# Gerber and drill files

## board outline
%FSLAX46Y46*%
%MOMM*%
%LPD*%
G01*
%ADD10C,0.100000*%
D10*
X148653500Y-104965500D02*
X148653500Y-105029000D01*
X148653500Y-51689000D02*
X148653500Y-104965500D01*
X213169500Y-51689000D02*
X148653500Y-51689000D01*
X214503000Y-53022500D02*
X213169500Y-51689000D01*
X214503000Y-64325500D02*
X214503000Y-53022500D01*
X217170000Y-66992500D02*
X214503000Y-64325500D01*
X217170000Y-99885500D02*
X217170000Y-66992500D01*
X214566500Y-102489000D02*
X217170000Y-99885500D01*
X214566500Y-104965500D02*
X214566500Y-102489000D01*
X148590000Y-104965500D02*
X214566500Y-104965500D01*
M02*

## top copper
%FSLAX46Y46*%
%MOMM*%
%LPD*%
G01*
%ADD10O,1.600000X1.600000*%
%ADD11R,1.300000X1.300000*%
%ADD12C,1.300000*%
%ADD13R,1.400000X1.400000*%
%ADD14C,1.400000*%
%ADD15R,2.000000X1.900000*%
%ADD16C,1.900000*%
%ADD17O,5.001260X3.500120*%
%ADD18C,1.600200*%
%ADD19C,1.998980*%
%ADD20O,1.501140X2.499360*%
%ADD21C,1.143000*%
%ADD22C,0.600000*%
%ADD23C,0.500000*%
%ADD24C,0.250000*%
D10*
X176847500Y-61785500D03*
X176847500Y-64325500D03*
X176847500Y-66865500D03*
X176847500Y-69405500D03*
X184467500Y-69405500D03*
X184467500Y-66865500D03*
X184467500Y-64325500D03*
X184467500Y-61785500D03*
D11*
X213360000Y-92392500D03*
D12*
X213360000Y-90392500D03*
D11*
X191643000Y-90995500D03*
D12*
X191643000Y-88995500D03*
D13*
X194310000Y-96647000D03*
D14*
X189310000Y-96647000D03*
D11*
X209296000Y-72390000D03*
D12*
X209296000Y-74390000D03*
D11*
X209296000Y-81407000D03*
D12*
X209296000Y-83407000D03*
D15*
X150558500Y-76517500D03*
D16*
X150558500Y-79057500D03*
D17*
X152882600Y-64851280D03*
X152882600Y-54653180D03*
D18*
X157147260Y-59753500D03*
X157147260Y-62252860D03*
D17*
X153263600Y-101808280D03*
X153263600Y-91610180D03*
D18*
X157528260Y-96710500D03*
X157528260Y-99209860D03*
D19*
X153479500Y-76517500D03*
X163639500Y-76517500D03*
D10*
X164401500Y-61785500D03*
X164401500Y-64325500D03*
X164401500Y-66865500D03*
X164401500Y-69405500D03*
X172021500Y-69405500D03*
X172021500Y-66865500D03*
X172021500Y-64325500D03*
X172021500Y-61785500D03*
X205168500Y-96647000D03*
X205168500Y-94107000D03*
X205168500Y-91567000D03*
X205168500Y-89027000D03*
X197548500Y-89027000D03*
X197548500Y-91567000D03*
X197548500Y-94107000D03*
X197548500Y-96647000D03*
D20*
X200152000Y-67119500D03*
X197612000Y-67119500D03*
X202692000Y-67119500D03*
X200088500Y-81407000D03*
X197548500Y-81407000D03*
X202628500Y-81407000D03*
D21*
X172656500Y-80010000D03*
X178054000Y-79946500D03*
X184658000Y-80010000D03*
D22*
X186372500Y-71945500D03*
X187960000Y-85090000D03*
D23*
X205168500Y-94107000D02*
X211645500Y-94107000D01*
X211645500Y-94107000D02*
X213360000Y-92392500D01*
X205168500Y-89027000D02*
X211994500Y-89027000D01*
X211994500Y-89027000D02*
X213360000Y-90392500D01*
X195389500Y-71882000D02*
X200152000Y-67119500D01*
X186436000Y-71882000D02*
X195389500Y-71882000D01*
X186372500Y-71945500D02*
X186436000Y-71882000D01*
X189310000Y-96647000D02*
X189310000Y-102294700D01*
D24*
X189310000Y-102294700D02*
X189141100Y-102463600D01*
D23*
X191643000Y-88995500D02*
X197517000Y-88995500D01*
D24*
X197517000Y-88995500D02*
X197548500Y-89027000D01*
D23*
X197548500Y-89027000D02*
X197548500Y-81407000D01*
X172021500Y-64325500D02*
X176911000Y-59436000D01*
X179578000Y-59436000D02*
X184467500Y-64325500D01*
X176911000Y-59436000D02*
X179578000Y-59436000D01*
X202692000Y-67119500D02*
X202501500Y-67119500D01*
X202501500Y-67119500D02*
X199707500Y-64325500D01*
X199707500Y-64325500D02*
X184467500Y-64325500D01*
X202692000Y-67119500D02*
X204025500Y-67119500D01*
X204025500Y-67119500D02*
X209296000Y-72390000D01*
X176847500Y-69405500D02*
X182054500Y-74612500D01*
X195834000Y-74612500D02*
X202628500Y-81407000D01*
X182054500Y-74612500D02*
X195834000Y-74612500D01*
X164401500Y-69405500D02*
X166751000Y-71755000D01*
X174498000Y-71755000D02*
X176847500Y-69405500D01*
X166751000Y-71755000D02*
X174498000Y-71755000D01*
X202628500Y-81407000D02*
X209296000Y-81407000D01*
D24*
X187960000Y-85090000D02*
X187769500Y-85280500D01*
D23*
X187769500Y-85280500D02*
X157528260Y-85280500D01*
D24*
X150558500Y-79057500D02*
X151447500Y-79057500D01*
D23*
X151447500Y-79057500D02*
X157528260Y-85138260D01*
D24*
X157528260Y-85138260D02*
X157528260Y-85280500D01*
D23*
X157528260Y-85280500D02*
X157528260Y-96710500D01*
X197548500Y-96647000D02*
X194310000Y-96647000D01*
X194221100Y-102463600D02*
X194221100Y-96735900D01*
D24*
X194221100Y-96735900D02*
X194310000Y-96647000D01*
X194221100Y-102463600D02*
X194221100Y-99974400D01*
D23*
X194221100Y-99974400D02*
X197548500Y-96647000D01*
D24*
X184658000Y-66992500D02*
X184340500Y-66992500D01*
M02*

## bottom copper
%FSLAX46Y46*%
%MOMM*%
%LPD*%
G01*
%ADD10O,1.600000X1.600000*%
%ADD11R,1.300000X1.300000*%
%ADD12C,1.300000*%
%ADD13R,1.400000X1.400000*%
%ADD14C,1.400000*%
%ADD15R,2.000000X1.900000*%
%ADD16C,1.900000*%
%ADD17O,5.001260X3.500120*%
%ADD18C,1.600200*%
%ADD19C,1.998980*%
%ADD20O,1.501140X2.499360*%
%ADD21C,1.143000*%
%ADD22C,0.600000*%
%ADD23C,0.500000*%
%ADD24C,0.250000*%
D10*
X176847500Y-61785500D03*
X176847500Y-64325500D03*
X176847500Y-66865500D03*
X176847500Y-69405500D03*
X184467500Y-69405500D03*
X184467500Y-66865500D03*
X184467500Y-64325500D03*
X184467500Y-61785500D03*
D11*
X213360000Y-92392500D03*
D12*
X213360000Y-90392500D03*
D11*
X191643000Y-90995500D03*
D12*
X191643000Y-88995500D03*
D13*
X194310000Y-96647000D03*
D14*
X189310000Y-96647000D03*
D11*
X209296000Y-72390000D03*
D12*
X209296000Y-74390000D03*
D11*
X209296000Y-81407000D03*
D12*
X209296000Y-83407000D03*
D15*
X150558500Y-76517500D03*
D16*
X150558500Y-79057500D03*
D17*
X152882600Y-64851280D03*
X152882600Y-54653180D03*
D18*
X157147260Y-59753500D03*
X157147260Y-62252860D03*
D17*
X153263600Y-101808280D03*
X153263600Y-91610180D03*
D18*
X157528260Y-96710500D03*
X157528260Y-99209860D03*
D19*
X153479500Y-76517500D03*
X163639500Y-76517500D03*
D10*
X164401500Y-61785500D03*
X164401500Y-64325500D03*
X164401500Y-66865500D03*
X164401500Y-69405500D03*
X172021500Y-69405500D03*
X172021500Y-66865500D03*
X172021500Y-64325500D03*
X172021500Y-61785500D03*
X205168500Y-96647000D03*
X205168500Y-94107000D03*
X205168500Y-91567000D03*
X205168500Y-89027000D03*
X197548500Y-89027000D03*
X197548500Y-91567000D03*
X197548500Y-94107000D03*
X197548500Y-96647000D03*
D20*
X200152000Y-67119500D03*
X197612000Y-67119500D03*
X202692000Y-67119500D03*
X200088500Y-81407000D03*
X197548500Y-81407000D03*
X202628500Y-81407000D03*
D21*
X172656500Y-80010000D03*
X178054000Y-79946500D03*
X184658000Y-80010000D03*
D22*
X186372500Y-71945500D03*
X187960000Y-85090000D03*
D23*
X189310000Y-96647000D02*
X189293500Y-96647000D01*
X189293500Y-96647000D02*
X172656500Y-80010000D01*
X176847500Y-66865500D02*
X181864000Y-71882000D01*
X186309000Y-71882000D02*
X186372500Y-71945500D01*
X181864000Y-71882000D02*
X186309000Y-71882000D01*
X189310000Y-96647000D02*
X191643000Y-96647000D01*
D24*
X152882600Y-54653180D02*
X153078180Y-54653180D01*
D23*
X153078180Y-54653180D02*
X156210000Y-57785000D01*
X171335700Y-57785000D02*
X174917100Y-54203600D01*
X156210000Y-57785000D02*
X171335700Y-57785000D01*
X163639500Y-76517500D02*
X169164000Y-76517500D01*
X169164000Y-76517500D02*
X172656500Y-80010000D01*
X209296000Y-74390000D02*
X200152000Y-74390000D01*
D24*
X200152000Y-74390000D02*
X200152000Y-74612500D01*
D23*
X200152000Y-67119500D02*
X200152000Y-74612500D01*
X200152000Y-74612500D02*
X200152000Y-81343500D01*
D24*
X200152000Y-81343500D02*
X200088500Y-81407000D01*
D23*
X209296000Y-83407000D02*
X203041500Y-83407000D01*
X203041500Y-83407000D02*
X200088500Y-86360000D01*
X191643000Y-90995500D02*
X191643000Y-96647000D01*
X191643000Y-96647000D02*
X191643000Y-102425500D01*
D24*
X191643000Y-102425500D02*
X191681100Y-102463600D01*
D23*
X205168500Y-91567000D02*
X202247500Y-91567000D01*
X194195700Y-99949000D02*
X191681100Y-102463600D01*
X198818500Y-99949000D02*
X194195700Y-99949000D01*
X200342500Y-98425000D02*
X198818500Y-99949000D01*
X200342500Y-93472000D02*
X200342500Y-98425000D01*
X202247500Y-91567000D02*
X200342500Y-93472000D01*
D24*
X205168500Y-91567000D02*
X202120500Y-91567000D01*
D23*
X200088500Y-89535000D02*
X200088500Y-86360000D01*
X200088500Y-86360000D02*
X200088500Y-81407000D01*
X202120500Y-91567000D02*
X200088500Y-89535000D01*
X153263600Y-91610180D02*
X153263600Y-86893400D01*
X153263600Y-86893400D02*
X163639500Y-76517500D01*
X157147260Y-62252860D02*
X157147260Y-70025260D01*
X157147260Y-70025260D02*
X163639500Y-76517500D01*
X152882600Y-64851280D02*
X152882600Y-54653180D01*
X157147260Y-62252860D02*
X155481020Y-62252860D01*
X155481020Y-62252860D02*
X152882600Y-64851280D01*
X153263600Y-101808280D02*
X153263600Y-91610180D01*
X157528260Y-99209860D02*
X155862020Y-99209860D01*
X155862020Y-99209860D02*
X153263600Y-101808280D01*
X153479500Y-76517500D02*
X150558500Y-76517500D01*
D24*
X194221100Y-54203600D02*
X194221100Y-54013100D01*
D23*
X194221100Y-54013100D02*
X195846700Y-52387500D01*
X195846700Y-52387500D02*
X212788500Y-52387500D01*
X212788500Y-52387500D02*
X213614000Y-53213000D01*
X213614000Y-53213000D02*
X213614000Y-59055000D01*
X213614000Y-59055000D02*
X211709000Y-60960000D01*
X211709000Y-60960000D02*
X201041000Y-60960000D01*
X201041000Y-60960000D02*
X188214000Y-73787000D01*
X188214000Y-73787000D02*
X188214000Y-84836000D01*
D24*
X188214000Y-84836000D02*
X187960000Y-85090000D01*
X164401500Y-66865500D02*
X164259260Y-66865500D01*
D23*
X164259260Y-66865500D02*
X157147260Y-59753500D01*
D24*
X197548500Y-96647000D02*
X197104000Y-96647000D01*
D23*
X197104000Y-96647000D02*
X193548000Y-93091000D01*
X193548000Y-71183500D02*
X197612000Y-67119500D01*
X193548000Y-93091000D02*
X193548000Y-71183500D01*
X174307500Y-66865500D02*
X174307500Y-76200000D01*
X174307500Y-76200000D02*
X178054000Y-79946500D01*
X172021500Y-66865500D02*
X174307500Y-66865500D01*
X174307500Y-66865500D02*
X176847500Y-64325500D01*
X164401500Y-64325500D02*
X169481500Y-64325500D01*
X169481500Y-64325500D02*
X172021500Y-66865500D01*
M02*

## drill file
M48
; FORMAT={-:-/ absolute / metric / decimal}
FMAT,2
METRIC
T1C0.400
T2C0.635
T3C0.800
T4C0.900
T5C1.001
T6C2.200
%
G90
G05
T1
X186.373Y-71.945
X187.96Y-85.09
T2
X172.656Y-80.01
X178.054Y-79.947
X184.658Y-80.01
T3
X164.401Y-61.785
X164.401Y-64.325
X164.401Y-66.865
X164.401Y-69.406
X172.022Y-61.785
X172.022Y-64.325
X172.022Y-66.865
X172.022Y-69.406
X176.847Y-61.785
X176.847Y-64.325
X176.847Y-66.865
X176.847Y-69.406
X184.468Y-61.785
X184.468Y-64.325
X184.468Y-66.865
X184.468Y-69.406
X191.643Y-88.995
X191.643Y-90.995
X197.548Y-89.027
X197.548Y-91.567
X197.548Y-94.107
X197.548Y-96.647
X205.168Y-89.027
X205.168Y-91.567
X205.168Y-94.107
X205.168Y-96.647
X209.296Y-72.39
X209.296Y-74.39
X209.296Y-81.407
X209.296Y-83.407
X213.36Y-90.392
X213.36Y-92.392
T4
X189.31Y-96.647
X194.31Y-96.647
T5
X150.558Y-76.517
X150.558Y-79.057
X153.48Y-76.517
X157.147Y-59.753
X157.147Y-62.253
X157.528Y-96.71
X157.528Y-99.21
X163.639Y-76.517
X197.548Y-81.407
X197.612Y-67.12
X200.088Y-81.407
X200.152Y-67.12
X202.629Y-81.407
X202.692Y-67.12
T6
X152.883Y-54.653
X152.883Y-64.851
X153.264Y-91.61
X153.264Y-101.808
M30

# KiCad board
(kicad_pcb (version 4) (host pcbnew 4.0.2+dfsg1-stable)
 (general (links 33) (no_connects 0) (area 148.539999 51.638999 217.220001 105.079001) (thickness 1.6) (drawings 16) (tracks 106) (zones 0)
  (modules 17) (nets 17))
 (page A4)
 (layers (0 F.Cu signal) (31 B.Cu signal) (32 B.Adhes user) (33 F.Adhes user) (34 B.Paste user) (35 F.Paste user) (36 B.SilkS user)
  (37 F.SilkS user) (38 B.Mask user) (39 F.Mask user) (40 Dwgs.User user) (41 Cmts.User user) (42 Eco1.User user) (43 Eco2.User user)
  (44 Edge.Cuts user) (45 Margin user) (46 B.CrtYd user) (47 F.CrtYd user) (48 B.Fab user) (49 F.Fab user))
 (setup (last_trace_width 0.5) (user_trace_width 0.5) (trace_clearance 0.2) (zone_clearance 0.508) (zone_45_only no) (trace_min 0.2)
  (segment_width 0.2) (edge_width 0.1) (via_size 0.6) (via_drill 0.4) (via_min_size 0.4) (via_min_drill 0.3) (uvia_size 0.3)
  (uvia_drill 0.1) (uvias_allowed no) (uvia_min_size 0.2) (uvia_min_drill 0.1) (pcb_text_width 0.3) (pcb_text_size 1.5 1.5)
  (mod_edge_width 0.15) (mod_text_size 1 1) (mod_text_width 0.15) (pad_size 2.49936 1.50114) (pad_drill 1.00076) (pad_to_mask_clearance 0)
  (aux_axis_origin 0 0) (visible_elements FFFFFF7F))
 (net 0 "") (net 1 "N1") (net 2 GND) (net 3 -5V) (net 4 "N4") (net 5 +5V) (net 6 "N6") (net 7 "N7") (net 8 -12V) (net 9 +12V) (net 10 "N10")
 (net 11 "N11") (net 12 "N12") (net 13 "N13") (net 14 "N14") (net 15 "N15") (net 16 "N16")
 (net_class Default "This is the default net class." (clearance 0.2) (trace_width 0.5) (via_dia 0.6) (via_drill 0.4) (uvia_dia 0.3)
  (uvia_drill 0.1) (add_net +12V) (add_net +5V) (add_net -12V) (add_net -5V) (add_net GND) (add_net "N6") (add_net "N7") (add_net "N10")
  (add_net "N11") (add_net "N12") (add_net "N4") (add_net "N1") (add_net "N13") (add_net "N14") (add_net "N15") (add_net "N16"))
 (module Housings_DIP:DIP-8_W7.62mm (layer F.Cu) (at 176.8475 61.7855)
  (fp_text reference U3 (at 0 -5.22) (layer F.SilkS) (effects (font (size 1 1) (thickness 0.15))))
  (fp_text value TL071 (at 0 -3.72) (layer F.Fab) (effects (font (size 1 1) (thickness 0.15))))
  (pad 1 thru_hole oval (at 0 0) (size 1.6 1.6) (drill 0.8) (layers *.Cu *.Mask F.SilkS))
  (pad 2 thru_hole oval (at 0 2.54) (size 1.6 1.6) (drill 0.8) (layers *.Cu *.Mask F.SilkS) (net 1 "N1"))
  (pad 3 thru_hole oval (at 0 5.08) (size 1.6 1.6) (drill 0.8) (layers *.Cu *.Mask F.SilkS) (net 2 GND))
  (pad 4 thru_hole oval (at 0 7.62) (size 1.6 1.6) (drill 0.8) (layers *.Cu *.Mask F.SilkS) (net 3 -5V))
  (pad 5 thru_hole oval (at 7.62 7.62) (size 1.6 1.6) (drill 0.8) (layers *.Cu *.Mask F.SilkS))
  (pad 6 thru_hole oval (at 7.62 5.08) (size 1.6 1.6) (drill 0.8) (layers *.Cu *.Mask F.SilkS) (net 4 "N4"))
  (pad 7 thru_hole oval (at 7.62 2.54) (size 1.6 1.6) (drill 0.8) (layers *.Cu *.Mask F.SilkS) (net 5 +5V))
  (pad 8 thru_hole oval (at 7.62 0) (size 1.6 1.6) (drill 0.8) (layers *.Cu *.Mask F.SilkS)))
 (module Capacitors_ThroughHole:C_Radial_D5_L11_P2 (layer F.Cu) (at 213.36 92.3925 90)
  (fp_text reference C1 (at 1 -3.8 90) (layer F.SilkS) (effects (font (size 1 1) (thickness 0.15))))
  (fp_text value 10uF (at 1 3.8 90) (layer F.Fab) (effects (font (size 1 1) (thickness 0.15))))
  (pad 1 thru_hole rect (at 0 0 90) (size 1.3 1.3) (drill 0.8) (layers *.Cu *.Mask F.SilkS) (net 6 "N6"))
  (pad 2 thru_hole circle (at 2 0 90) (size 1.3 1.3) (drill 0.8) (layers *.Cu *.Mask F.SilkS) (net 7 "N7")))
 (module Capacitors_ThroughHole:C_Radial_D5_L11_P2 (layer F.Cu) (at 191.643 90.9955 90)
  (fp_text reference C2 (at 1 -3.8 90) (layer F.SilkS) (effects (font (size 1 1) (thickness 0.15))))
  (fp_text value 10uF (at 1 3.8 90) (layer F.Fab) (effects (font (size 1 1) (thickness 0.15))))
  (pad 1 thru_hole rect (at 0 0 90) (size 1.3 1.3) (drill 0.8) (layers *.Cu *.Mask F.SilkS) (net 2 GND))
  (pad 2 thru_hole circle (at 2 0 90) (size 1.3 1.3) (drill 0.8) (layers *.Cu *.Mask F.SilkS) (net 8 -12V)))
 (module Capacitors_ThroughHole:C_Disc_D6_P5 (layer F.Cu) (at 194.31 96.647 180)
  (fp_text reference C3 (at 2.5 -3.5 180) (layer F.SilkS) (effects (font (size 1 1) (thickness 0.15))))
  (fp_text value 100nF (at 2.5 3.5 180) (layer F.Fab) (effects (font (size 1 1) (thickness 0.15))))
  (pad 1 thru_hole rect (at 0 0 180) (size 1.4 1.4) (drill 0.9) (layers *.Cu *.Mask F.SilkS) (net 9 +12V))
  (pad 2 thru_hole circle (at 5 0 180) (size 1.4 1.4) (drill 0.9) (layers *.Cu *.Mask F.SilkS) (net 2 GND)))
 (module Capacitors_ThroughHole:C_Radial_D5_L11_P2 (layer F.Cu) (at 209.296 72.39 270)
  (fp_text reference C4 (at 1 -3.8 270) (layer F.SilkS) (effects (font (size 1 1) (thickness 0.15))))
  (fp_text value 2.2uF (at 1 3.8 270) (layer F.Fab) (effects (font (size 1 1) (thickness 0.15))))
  (pad 1 thru_hole rect (at 0 0 270) (size 1.3 1.3) (drill 0.8) (layers *.Cu *.Mask F.SilkS) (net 5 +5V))
  (pad 2 thru_hole circle (at 2 0 270) (size 1.3 1.3) (drill 0.8) (layers *.Cu *.Mask F.SilkS) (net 2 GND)))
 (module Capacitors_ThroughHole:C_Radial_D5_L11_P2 (layer F.Cu) (at 209.296 81.407 270)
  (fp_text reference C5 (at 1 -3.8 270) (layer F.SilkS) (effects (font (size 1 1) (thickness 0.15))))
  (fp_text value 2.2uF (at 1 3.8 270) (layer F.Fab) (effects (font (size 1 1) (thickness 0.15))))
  (pad 1 thru_hole rect (at 0 0 270) (size 1.3 1.3) (drill 0.8) (layers *.Cu *.Mask F.SilkS) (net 3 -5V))
  (pad 2 thru_hole circle (at 2 0 270) (size 1.3 1.3) (drill 0.8) (layers *.Cu *.Mask F.SilkS) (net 2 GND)))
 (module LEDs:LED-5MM (layer F.Cu) (at 150.5585 76.5175 270)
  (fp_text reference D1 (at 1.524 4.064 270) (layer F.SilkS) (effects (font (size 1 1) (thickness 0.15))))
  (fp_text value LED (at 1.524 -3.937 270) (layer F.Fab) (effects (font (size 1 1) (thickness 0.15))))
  (pad 1 thru_hole rect (at 0 0) (size 2 1.9) (drill 1.00076) (layers *.Cu *.Mask F.SilkS) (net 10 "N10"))
  (pad 2 thru_hole circle (at 2.54 0 270) (size 1.9 1.9) (drill 1.00076) (layers *.Cu *.Mask F.SilkS) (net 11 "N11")))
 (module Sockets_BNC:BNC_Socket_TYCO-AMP (layer F.Cu) (at 152.146 59.7535 90)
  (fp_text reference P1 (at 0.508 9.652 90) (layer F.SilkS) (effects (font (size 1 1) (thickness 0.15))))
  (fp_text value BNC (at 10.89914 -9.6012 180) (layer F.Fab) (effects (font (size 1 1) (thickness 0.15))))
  (pad 2 thru_hole oval (at -5.09778 0.7366 90) (size 3.50012 5.00126) (drill 2.19964) (layers *.Cu *.Mask F.SilkS) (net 2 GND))
  (pad 2 thru_hole oval (at 5.10032 0.7366 90) (size 3.50012 5.00126) (drill 2.19964) (layers *.Cu *.Mask F.SilkS) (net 2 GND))
  (pad 1 thru_hole circle (at 0 5.00126 90) (size 1.6002 1.6002) (drill 1.00076) (layers *.Cu *.Mask F.SilkS) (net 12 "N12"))
  (pad 2 thru_hole circle (at -2.49936 5.00126 90) (size 1.6002 1.6002) (drill 1.00076) (layers *.Cu *.Mask F.SilkS) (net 2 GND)))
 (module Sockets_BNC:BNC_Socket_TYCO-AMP (layer F.Cu) (at 152.527 96.7105 90)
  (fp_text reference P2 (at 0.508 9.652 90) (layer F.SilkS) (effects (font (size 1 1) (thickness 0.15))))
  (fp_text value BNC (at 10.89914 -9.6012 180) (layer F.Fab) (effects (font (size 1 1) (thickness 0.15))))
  (pad 2 thru_hole oval (at -5.09778 0.7366 90) (size 3.50012 5.00126) (drill 2.19964) (layers *.Cu *.Mask F.SilkS) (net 2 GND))
  (pad 2 thru_hole oval (at 5.10032 0.7366 90) (size 3.50012 5.00126) (drill 2.19964) (layers *.Cu *.Mask F.SilkS) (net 2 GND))
  (pad 1 thru_hole circle (at 0 5.00126 90) (size 1.6002 1.6002) (drill 1.00076) (layers *.Cu *.Mask F.SilkS) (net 11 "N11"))
  (pad 2 thru_hole circle (at -2.49936 5.00126 90) (size 1.6002 1.6002) (drill 1.00076) (layers *.Cu *.Mask F.SilkS) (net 2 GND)))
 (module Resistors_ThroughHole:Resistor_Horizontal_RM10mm (layer F.Cu) (at 153.4795 76.5175)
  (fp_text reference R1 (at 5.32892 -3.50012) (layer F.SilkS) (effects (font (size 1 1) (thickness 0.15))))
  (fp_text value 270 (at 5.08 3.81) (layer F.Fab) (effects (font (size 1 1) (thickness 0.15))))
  (pad 1 thru_hole circle (at 0 0) (size 1.99898 1.99898) (drill 1.00076) (layers *.Cu *.SilkS *.Mask) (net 10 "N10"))
  (pad 2 thru_hole circle (at 10.16 0) (size 1.99898 1.99898) (drill 1.00076) (layers *.Cu *.SilkS *.Mask) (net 2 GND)))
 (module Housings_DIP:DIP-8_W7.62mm (layer F.Cu) (at 164.4015 61.7855)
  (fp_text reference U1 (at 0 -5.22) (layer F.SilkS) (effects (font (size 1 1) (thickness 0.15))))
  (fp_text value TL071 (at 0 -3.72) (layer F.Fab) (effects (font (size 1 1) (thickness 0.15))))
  (pad 1 thru_hole oval (at 0 0) (size 1.6 1.6) (drill 0.8) (layers *.Cu *.Mask F.SilkS))
  (pad 2 thru_hole oval (at 0 2.54) (size 1.6 1.6) (drill 0.8) (layers *.Cu *.Mask F.SilkS) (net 1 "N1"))
  (pad 3 thru_hole oval (at 0 5.08) (size 1.6 1.6) (drill 0.8) (layers *.Cu *.Mask F.SilkS) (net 12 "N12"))
  (pad 4 thru_hole oval (at 0 7.62) (size 1.6 1.6) (drill 0.8) (layers *.Cu *.Mask F.SilkS) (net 3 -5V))
  (pad 5 thru_hole oval (at 7.62 7.62) (size 1.6 1.6) (drill 0.8) (layers *.Cu *.Mask F.SilkS))
  (pad 6 thru_hole oval (at 7.62 5.08) (size 1.6 1.6) (drill 0.8) (layers *.Cu *.Mask F.SilkS) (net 1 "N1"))
  (pad 7 thru_hole oval (at 7.62 2.54) (size 1.6 1.6) (drill 0.8) (layers *.Cu *.Mask F.SilkS) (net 5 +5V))
  (pad 8 thru_hole oval (at 7.62 0) (size 1.6 1.6) (drill 0.8) (layers *.Cu *.Mask F.SilkS)))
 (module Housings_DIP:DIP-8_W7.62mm (layer F.Cu) (at 205.1685 96.647 180)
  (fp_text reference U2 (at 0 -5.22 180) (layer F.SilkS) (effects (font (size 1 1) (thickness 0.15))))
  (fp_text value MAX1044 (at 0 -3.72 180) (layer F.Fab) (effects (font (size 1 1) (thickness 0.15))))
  (pad 1 thru_hole oval (at 0 0 180) (size 1.6 1.6) (drill 0.8) (layers *.Cu *.Mask F.SilkS) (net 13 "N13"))
  (pad 2 thru_hole oval (at 0 2.54 180) (size 1.6 1.6) (drill 0.8) (layers *.Cu *.Mask F.SilkS) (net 6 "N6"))
  (pad 3 thru_hole oval (at 0 5.08 180) (size 1.6 1.6) (drill 0.8) (layers *.Cu *.Mask F.SilkS) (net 2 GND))
  (pad 4 thru_hole oval (at 0 7.62 180) (size 1.6 1.6) (drill 0.8) (layers *.Cu *.Mask F.SilkS) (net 7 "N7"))
  (pad 5 thru_hole oval (at 7.62 7.62 180) (size 1.6 1.6) (drill 0.8) (layers *.Cu *.Mask F.SilkS) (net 8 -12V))
  (pad 6 thru_hole oval (at 7.62 5.08 180) (size 1.6 1.6) (drill 0.8) (layers *.Cu *.Mask F.SilkS) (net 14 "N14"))
  (pad 7 thru_hole oval (at 7.62 2.54 180) (size 1.6 1.6) (drill 0.8) (layers *.Cu *.Mask F.SilkS) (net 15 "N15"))
  (pad 8 thru_hole oval (at 7.62 0 180) (size 1.6 1.6) (drill 0.8) (layers *.Cu *.Mask F.SilkS) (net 9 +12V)))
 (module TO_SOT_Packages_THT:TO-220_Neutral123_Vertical (layer F.Cu) (at 200.152 67.1195)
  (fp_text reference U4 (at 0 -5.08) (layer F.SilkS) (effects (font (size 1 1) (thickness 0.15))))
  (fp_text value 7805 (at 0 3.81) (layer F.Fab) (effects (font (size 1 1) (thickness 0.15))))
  (pad GND thru_hole oval (at 0 0 90) (size 2.49936 1.50114) (drill 1.00076) (layers *.Cu *.Mask F.SilkS) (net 2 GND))
  (pad VI thru_hole oval (at -2.54 0 90) (size 2.49936 1.50114) (drill 1.00076) (layers *.Cu *.Mask F.SilkS) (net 9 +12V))
  (pad VO thru_hole oval (at 2.54 0 90) (size 2.49936 1.50114) (drill 1.00076) (layers *.Cu *.Mask F.SilkS) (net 5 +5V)))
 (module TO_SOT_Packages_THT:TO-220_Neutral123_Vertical (layer F.Cu) (at 200.0885 81.407)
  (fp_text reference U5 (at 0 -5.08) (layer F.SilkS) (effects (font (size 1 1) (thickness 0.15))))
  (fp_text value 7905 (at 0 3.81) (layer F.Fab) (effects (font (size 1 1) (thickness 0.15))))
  (pad GND thru_hole oval (at 0 0 90) (size 2.49936 1.50114) (drill 1.00076) (layers *.Cu *.Mask F.SilkS) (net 2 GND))
  (pad VI thru_hole oval (at -2.54 0 90) (size 2.49936 1.50114) (drill 1.00076) (layers *.Cu *.Mask F.SilkS) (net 8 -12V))
  (pad VO thru_hole oval (at 2.54 0 90) (size 2.49936 1.50114) (drill 1.00076) (layers *.Cu *.Mask F.SilkS) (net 3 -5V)))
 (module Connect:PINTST (layer F.Cu) (at 172.6565 80.01)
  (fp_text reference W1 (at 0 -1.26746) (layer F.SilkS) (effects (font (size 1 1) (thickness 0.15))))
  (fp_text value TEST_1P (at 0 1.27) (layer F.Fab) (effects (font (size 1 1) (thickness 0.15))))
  (pad 1 thru_hole circle (at 0 0) (size 1.143 1.143) (drill 0.635) (layers *.Cu *.Mask F.SilkS) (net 2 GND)))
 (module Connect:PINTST (layer F.Cu) (at 178.054 79.9465)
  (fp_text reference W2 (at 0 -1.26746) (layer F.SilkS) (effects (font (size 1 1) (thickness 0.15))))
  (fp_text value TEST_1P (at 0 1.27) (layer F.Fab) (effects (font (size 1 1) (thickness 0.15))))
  (pad 1 thru_hole circle (at 0 0) (size 1.143 1.143) (drill 0.635) (layers *.Cu *.Mask F.SilkS) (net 1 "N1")))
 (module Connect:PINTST (layer F.Cu) (at 184.658 80.01)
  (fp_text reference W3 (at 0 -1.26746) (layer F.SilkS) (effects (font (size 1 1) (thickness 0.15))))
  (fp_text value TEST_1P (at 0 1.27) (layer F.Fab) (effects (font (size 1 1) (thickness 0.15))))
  (pad 1 thru_hole circle (at 0 0) (size 1.143 1.143) (drill 0.635) (layers *.Cu *.Mask F.SilkS) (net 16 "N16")))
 (gr_line (start 148.6535 104.9655) (end 148.6535 105.029) (angle 90) (layer Edge.Cuts) (width 0.1))
 (gr_line (start 148.6535 51.689) (end 148.6535 104.9655) (angle 90) (layer Edge.Cuts) (width 0.1))
 (gr_line (start 213.1695 51.689) (end 148.6535 51.689) (angle 90) (layer Edge.Cuts) (width 0.1))
 (gr_line (start 214.503 53.0225) (end 213.1695 51.689) (angle 90) (layer Edge.Cuts) (width 0.1))
 (gr_line (start 214.503 64.3255) (end 214.503 53.0225) (angle 90) (layer Edge.Cuts) (width 0.1))
 (gr_line (start 217.17 66.9925) (end 214.503 64.3255) (angle 90) (layer Edge.Cuts) (width 0.1))
 (gr_line (start 217.17 99.8855) (end 217.17 66.9925) (angle 90) (layer Edge.Cuts) (width 0.1))
 (gr_line (start 214.5665 102.489) (end 217.17 99.8855) (angle 90) (layer Edge.Cuts) (width 0.1))
 (gr_line (start 214.5665 104.9655) (end 214.5665 102.489) (angle 90) (layer Edge.Cuts) (width 0.1))
 (gr_line (start 148.59 104.9655) (end 214.5665 104.9655) (angle 90) (layer Edge.Cuts) (width 0.1))
 (segment (start 205.1685 94.107) (end 211.6455 94.107) (width 0.5) (layer F.Cu) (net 6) (status 10))
 (segment (start 211.6455 94.107) (end 213.36 92.3925) (width 0.5) (layer F.Cu) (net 6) (status 20))
 (segment (start 205.1685 89.027) (end 211.9945 89.027) (width 0.5) (layer F.Cu) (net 7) (status 10))
 (segment (start 211.9945 89.027) (end 213.36 90.3925) (width 0.5) (layer F.Cu) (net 7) (status 20))
 (segment (start 189.31 96.647) (end 189.2935 96.647) (width 0.5) (layer B.Cu) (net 2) (status C00000))
 (segment (start 189.2935 96.647) (end 172.6565 80.01) (width 0.5) (layer B.Cu) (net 2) (status C00000))
 (segment (start 176.8475 66.8655) (end 181.864 71.882) (width 0.5) (layer B.Cu) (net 2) (status 400000))
 (segment (start 195.3895 71.882) (end 200.152 67.1195) (width 0.5) (layer F.Cu) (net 2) (status 800000))
 (segment (start 186.436 71.882) (end 195.3895 71.882) (width 0.5) (layer F.Cu) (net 2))
 (segment (start 186.3725 71.9455) (end 186.436 71.882) (width 0.5) (layer F.Cu) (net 2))
 (via (at 186.3725 71.9455) (size 0.6) (drill 0.4) (layers F.Cu B.Cu) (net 2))
 (segment (start 186.309 71.882) (end 186.3725 71.9455) (width 0.5) (layer B.Cu) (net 2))
 (segment (start 181.864 71.882) (end 186.309 71.882) (width 0.5) (layer B.Cu) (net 2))
 (segment (start 189.31 96.647) (end 191.643 96.647) (width 0.5) (layer B.Cu) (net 2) (status 10))
 (segment (start 189.31 96.647) (end 189.31 102.2947) (width 0.5) (layer F.Cu) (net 2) (status 30))
 (segment (start 189.31 102.2947) (end 189.1411 102.4636) (width 0.25) (layer F.Cu) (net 2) (status 30))
 (segment (start 152.8826 54.65318) (end 153.07818 54.65318) (width 0.25) (layer B.Cu) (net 2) (status 30))
 (segment (start 153.07818 54.65318) (end 156.21 57.785) (width 0.5) (layer B.Cu) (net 2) (status 10))
 (segment (start 171.3357 57.785) (end 174.9171 54.2036) (width 0.5) (layer B.Cu) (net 2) (status 20))
 (segment (start 156.21 57.785) (end 171.3357 57.785) (width 0.5) (layer B.Cu) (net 2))
 (segment (start 163.6395 76.5175) (end 169.164 76.5175) (width 0.5) (layer B.Cu) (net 2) (status 10))
 (segment (start 169.164 76.5175) (end 172.6565 80.01) (width 0.5) (layer B.Cu) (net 2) (status 20))
 (segment (start 209.296 74.39) (end 200.152 74.39) (width 0.5) (layer B.Cu) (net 2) (status 10))
 (segment (start 200.152 74.39) (end 200.152 74.6125) (width 0.25) (layer B.Cu) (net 2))
 (segment (start 200.152 67.1195) (end 200.152 74.6125) (width 0.5) (layer B.Cu) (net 2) (status 10))
 (segment (start 200.152 74.6125) (end 200.152 81.3435) (width 0.5) (layer B.Cu) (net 2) (status 20))
 (segment (start 200.152 81.3435) (end 200.0885 81.407) (width 0.25) (layer B.Cu) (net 2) (status 30))
 (segment (start 209.296 83.407) (end 203.0415 83.407) (width 0.5) (layer B.Cu) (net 2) (status 10))
 (segment (start 203.0415 83.407) (end 200.0885 86.36) (width 0.5) (layer B.Cu) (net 2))
 (segment (start 191.643 90.9955) (end 191.643 96.647) (width 0.5) (layer B.Cu) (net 2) (status 10))
 (segment (start 191.643 96.647) (end 191.643 102.4255) (width 0.5) (layer B.Cu) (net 2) (status 20))
 (segment (start 191.643 102.4255) (end 191.6811 102.4636) (width 0.25) (layer B.Cu) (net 2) (status 30))
 (segment (start 205.1685 91.567) (end 202.2475 91.567) (width 0.5) (layer B.Cu) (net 2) (status 10))
 (segment (start 194.1957 99.949) (end 191.6811 102.4636) (width 0.5) (layer B.Cu) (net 2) (status 20))
 (segment (start 198.8185 99.949) (end 194.1957 99.949) (width 0.5) (layer B.Cu) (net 2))
 (segment (start 200.3425 98.425) (end 198.8185 99.949) (width 0.5) (layer B.Cu) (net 2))
 (segment (start 200.3425 93.472) (end 200.3425 98.425) (width 0.5) (layer B.Cu) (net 2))
 (segment (start 202.2475 91.567) (end 200.3425 93.472) (width 0.5) (layer B.Cu) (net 2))
 (segment (start 205.1685 91.567) (end 202.1205 91.567) (width 0.25) (layer B.Cu) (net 2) (status 10))
 (segment (start 200.0885 89.535) (end 200.0885 86.36) (width 0.5) (layer B.Cu) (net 2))
 (segment (start 200.0885 86.36) (end 200.0885 81.407) (width 0.5) (layer B.Cu) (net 2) (status 20))
 (segment (start 202.1205 91.567) (end 200.0885 89.535) (width 0.5) (layer B.Cu) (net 2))
 (segment (start 153.2636 91.61018) (end 153.2636 86.8934) (width 0.5) (layer B.Cu) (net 2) (status 10))
 (segment (start 153.2636 86.8934) (end 163.6395 76.5175) (width 0.5) (layer B.Cu) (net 2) (status 20))
 (segment (start 157.14726 62.25286) (end 157.14726 70.02526) (width 0.5) (layer B.Cu) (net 2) (status 10))
 (segment (start 157.14726 70.02526) (end 163.6395 76.5175) (width 0.5) (layer B.Cu) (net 2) (status 20))
 (segment (start 152.8826 64.85128) (end 152.8826 54.65318) (width 0.5) (layer B.Cu) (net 2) (status 30))
 (segment (start 157.14726 62.25286) (end 155.48102 62.25286) (width 0.5) (layer B.Cu) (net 2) (status 10))
 (segment (start 155.48102 62.25286) (end 152.8826 64.85128) (width 0.5) (layer B.Cu) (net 2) (status 20))
 (segment (start 153.2636 101.80828) (end 153.2636 91.61018) (width 0.5) (layer B.Cu) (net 2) (status 30))
 (segment (start 157.52826 99.20986) (end 155.86202 99.20986) (width 0.5) (layer B.Cu) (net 2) (status 10))
 (segment (start 155.86202 99.20986) (end 153.2636 101.80828) (width 0.5) (layer B.Cu) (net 2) (status 20))
 (segment (start 191.643 88.9955) (end 197.517 88.9955) (width 0.5) (layer F.Cu) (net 8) (status 30))
 (segment (start 197.517 88.9955) (end 197.5485 89.027) (width 0.25) (layer F.Cu) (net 8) (status 30))
 (segment (start 197.5485 89.027) (end 197.5485 81.407) (width 0.5) (layer F.Cu) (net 8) (status 30))
 (segment (start 172.0215 64.3255) (end 176.911 59.436) (width 0.5) (layer F.Cu) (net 5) (status 400000))
 (segment (start 179.578 59.436) (end 184.4675 64.3255) (width 0.5) (layer F.Cu) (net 5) (status 800000))
 (segment (start 176.911 59.436) (end 179.578 59.436) (width 0.5) (layer F.Cu) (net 5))
 (segment (start 202.692 67.1195) (end 202.5015 67.1195) (width 0.5) (layer F.Cu) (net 5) (status C00000))
 (segment (start 202.5015 67.1195) (end 199.7075 64.3255) (width 0.5) (layer F.Cu) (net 5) (status 400000))
 (segment (start 199.7075 64.3255) (end 184.4675 64.3255) (width 0.5) (layer F.Cu) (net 5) (status 800000))
 (segment (start 202.692 67.1195) (end 204.0255 67.1195) (width 0.5) (layer F.Cu) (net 5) (status 10))
 (segment (start 204.0255 67.1195) (end 209.296 72.39) (width 0.5) (layer F.Cu) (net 5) (status 20))
 (segment (start 176.8475 69.4055) (end 182.0545 74.6125) (width 0.5) (layer F.Cu) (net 3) (status 400000))
 (segment (start 195.834 74.6125) (end 202.6285 81.407) (width 0.5) (layer F.Cu) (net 3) (status 800000))
 (segment (start 182.0545 74.6125) (end 195.834 74.6125) (width 0.5) (layer F.Cu) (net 3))
 (segment (start 164.4015 69.4055) (end 166.751 71.755) (width 0.5) (layer F.Cu) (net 3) (status 400000))
 (segment (start 174.498 71.755) (end 176.8475 69.4055) (width 0.5) (layer F.Cu) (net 3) (status 800000))
 (segment (start 166.751 71.755) (end 174.498 71.755) (width 0.5) (layer F.Cu) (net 3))
 (segment (start 202.6285 81.407) (end 209.296 81.407) (width 0.5) (layer F.Cu) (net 3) (status 30))
 (segment (start 153.4795 76.5175) (end 150.5585 76.5175) (width 0.5) (layer B.Cu) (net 10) (status 30))
 (segment (start 194.2211 54.2036) (end 194.2211 54.0131) (width 0.25) (layer B.Cu) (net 11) (status 30))
 (segment (start 194.2211 54.0131) (end 195.8467 52.3875) (width 0.5) (layer B.Cu) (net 11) (status 10))
 (segment (start 195.8467 52.3875) (end 212.7885 52.3875) (width 0.5) (layer B.Cu) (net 11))
 (segment (start 212.7885 52.3875) (end 213.614 53.213) (width 0.5) (layer B.Cu) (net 11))
 (segment (start 213.614 53.213) (end 213.614 59.055) (width 0.5) (layer B.Cu) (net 11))
 (segment (start 213.614 59.055) (end 211.709 60.96) (width 0.5) (layer B.Cu) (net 11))
 (segment (start 211.709 60.96) (end 201.041 60.96) (width 0.5) (layer B.Cu) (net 11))
 (segment (start 201.041 60.96) (end 188.214 73.787) (width 0.5) (layer B.Cu) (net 11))
 (segment (start 188.214 73.787) (end 188.214 84.836) (width 0.5) (layer B.Cu) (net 11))
 (segment (start 188.214 84.836) (end 187.96 85.09) (width 0.25) (layer B.Cu) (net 11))
 (via (at 187.96 85.09) (size 0.6) (drill 0.4) (layers F.Cu B.Cu) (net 11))
 (segment (start 187.96 85.09) (end 187.7695 85.2805) (width 0.25) (layer F.Cu) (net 11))
 (segment (start 187.7695 85.2805) (end 157.52826 85.2805) (width 0.5) (layer F.Cu) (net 11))
 (segment (start 150.5585 79.0575) (end 151.4475 79.0575) (width 0.25) (layer F.Cu) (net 11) (status 30))
 (segment (start 151.4475 79.0575) (end 157.52826 85.13826) (width 0.5) (layer F.Cu) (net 11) (status 10))
 (segment (start 157.52826 85.13826) (end 157.52826 85.2805) (width 0.25) (layer F.Cu) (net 11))
 (segment (start 157.52826 85.2805) (end 157.52826 96.7105) (width 0.5) (layer F.Cu) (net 11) (status 20))
 (segment (start 164.4015 66.8655) (end 164.25926 66.8655) (width 0.25) (layer B.Cu) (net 12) (status 30))
 (segment (start 164.25926 66.8655) (end 157.14726 59.7535) (width 0.5) (layer B.Cu) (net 12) (status 30))
 (segment (start 197.5485 96.647) (end 194.31 96.647) (width 0.5) (layer F.Cu) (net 9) (status 30))
 (segment (start 194.2211 102.4636) (end 194.2211 96.7359) (width 0.5) (layer F.Cu) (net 9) (status 30))
 (segment (start 194.2211 96.7359) (end 194.31 96.647) (width 0.25) (layer F.Cu) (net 9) (status 30))
 (segment (start 197.5485 96.647) (end 197.104 96.647) (width 0.25) (layer B.Cu) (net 9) (status 30))
 (segment (start 197.104 96.647) (end 193.548 93.091) (width 0.5) (layer B.Cu) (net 9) (status 10))
 (segment (start 193.548 71.1835) (end 197.612 67.1195) (width 0.5) (layer B.Cu) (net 9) (status 20))
 (segment (start 193.548 93.091) (end 193.548 71.1835) (width 0.5) (layer B.Cu) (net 9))
 (segment (start 194.2211 102.4636) (end 194.2211 99.9744) (width 0.25) (layer F.Cu) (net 9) (status 10))
 (segment (start 194.2211 99.9744) (end 197.5485 96.647) (width 0.5) (layer F.Cu) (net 9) (status 20))
 (segment (start 184.658 66.9925) (end 184.3405 66.9925) (width 0.25) (layer F.Cu) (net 4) (status 30))
 (segment (start 174.3075 66.8655) (end 174.3075 76.2) (width 0.5) (layer B.Cu) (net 1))
 (segment (start 174.3075 76.2) (end 178.054 79.9465) (width 0.5) (layer B.Cu) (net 1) (status 800000))
 (segment (start 172.0215 66.8655) (end 174.3075 66.8655) (width 0.5) (layer B.Cu) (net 1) (status 400000))
 (segment (start 174.3075 66.8655) (end 176.8475 64.3255) (width 0.5) (layer B.Cu) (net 1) (status 800000))
 (segment (start 164.4015 64.3255) (end 169.4815 64.3255) (width 0.5) (layer B.Cu) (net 1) (status 10))
 (segment (start 169.4815 64.3255) (end 172.0215 66.8655) (width 0.5) (layer B.Cu) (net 1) (status 20)))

